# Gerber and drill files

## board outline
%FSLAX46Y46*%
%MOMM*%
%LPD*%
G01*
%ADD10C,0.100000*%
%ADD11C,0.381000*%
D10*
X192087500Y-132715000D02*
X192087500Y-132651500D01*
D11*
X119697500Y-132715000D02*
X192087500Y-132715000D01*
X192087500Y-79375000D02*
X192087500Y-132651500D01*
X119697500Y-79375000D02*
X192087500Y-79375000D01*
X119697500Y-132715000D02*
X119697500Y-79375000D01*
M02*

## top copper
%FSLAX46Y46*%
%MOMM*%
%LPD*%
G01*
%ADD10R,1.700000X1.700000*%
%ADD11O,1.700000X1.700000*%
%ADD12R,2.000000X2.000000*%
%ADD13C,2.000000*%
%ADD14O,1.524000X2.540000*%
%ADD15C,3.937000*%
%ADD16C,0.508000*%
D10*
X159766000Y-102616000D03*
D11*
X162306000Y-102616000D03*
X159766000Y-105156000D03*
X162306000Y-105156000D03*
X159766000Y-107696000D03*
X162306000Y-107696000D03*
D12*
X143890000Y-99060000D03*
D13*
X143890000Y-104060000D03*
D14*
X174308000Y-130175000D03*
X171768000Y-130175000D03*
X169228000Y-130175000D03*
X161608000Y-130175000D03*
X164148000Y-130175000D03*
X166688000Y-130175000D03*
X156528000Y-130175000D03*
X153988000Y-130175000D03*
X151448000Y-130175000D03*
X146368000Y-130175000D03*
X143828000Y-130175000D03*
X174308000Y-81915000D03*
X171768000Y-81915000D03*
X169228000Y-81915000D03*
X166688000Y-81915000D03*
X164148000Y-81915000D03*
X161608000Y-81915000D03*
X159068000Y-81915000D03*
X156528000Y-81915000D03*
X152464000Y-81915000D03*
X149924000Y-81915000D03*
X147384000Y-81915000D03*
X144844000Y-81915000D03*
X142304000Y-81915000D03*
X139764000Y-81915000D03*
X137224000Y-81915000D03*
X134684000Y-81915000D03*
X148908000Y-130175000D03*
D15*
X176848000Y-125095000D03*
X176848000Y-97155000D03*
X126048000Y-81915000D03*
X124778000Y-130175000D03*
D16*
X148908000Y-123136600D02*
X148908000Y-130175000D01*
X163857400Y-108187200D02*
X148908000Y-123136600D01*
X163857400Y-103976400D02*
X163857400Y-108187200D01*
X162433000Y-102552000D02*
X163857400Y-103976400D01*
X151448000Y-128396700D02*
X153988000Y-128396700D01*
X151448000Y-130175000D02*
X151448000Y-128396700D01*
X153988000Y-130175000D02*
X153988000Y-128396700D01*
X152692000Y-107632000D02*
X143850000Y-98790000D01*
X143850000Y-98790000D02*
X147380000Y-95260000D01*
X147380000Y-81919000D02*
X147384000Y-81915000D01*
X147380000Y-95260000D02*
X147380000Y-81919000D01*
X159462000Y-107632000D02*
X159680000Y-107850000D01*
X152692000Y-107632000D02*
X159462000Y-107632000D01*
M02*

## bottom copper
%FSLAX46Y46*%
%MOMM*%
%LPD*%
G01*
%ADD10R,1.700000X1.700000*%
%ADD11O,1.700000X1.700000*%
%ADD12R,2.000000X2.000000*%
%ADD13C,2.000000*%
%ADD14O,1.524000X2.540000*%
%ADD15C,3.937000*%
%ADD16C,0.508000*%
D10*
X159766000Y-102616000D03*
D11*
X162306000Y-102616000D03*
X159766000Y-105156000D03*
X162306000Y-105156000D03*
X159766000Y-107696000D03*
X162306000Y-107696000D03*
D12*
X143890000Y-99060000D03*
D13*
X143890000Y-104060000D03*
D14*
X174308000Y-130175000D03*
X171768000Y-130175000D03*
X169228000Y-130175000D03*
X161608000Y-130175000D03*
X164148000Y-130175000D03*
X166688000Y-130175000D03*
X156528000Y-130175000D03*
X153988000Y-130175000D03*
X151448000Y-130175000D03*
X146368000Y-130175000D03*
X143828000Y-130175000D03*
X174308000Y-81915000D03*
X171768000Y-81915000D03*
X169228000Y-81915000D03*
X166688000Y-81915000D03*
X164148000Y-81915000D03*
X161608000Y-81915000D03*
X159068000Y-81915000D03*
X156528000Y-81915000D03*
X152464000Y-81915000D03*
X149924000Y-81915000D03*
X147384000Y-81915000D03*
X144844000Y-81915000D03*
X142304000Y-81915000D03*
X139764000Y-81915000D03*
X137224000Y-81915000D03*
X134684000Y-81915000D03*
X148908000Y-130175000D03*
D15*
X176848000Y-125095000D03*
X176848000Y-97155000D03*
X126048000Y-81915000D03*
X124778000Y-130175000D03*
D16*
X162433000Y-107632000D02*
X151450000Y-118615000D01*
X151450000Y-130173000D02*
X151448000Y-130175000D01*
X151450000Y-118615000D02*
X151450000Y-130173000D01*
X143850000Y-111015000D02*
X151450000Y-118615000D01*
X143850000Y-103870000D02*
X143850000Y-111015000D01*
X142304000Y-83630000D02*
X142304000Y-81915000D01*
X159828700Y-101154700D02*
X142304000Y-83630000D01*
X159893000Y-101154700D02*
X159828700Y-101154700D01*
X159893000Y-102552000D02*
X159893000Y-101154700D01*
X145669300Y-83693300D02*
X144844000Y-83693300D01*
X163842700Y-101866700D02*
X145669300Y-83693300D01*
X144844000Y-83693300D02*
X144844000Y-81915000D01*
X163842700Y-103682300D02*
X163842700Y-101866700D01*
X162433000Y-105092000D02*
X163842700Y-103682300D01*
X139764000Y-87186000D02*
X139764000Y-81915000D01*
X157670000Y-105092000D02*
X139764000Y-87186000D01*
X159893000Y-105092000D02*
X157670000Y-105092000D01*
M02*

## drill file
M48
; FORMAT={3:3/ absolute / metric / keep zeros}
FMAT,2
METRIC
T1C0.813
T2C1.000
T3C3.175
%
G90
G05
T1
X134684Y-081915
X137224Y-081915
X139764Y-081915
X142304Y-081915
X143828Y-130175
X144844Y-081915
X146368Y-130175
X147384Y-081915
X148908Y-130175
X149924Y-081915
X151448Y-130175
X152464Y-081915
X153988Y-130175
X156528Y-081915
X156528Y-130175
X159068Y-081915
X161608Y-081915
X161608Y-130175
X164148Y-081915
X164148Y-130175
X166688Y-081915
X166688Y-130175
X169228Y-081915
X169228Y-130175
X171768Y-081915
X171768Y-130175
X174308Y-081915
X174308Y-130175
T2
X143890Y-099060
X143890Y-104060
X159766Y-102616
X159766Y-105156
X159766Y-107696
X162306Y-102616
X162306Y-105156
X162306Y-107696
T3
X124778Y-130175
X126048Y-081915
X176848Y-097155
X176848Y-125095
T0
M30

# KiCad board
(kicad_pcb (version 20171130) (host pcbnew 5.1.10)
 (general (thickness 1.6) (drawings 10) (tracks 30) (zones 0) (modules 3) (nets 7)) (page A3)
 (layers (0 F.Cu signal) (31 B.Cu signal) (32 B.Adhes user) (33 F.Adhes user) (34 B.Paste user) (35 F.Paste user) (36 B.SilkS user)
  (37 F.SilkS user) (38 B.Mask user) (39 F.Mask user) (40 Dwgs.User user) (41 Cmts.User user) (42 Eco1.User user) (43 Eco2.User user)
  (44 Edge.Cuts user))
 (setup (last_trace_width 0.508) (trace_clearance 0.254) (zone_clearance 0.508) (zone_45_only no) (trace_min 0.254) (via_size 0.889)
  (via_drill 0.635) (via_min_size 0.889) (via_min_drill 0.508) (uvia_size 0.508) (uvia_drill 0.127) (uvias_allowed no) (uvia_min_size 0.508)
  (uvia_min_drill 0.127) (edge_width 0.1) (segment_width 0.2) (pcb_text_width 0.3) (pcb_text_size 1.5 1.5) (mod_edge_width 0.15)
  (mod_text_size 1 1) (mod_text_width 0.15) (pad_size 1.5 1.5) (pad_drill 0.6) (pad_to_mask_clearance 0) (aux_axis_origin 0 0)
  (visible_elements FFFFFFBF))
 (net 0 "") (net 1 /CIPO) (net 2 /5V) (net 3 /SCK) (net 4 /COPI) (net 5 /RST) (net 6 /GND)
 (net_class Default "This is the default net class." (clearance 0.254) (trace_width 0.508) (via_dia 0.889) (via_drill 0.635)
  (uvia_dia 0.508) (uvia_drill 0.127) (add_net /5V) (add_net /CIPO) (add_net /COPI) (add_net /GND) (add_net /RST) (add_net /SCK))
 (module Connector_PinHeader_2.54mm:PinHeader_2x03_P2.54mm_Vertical (layer F.Cu) (at 159.766 102.616)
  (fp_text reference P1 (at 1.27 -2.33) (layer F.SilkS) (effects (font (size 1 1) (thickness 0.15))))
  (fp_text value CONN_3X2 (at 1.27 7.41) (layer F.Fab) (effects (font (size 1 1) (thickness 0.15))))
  (pad 1 thru_hole rect (at 0 0) (size 1.7 1.7) (drill 1) (layers *.Cu *.Mask) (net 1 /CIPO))
  (pad 2 thru_hole oval (at 2.54 0) (size 1.7 1.7) (drill 1) (layers *.Cu *.Mask) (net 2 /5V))
  (pad 3 thru_hole oval (at 0 2.54) (size 1.7 1.7) (drill 1) (layers *.Cu *.Mask) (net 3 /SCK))
  (pad 4 thru_hole oval (at 2.54 2.54) (size 1.7 1.7) (drill 1) (layers *.Cu *.Mask) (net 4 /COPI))
  (pad 5 thru_hole oval (at 0 5.08) (size 1.7 1.7) (drill 1) (layers *.Cu *.Mask) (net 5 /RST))
  (pad 6 thru_hole oval (at 2.54 5.08) (size 1.7 1.7) (drill 1) (layers *.Cu *.Mask) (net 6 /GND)))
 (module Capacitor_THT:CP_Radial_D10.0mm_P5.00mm (layer F.Cu) (at 143.89 99.06 270)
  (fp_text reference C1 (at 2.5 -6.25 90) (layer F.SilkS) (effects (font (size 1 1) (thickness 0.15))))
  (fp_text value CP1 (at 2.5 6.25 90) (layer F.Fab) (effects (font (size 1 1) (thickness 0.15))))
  (pad 1 thru_hole rect (at 0 0 270) (size 2 2) (drill 1) (layers *.Cu *.Mask) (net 5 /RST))
  (pad 2 thru_hole circle (at 5 0 270) (size 2 2) (drill 1) (layers *.Cu *.Mask) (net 6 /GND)))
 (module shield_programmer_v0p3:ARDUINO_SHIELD (layer F.Cu) (at 119.698 132.715)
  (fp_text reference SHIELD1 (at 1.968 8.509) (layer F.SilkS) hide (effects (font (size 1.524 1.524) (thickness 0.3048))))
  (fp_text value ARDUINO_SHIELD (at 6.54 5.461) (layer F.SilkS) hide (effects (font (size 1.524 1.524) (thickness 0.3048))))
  (pad AD5 thru_hole oval (at 54.61 -2.54 90) (size 2.54 1.524) (drill 0.8128) (layers *.Cu *.Mask F.SilkS))
  (pad AD4 thru_hole oval (at 52.07 -2.54 90) (size 2.54 1.524) (drill 0.8128) (layers *.Cu *.Mask F.SilkS))
  (pad AD3 thru_hole oval (at 49.53 -2.54 90) (size 2.54 1.524) (drill 0.8128) (layers *.Cu *.Mask F.SilkS))
  (pad AD0 thru_hole oval (at 41.91 -2.54 90) (size 2.54 1.524) (drill 0.8128) (layers *.Cu *.Mask F.SilkS))
  (pad AD1 thru_hole oval (at 44.45 -2.54 90) (size 2.54 1.524) (drill 0.8128) (layers *.Cu *.Mask F.SilkS))
  (pad AD2 thru_hole oval (at 46.99 -2.54 90) (size 2.54 1.524) (drill 0.8128) (layers *.Cu *.Mask F.SilkS))
  (pad V_IN thru_hole oval (at 36.83 -2.54 90) (size 2.54 1.524) (drill 0.8128) (layers *.Cu *.Mask F.SilkS))
  (pad GND2 thru_hole oval (at 34.29 -2.54 90) (size 2.54 1.524) (drill 0.8128) (layers *.Cu *.Mask F.SilkS) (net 6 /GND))
  (pad GND1 thru_hole oval (at 31.75 -2.54 90) (size 2.54 1.524) (drill 0.8128) (layers *.Cu *.Mask F.SilkS) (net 6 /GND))
  (pad 3V3 thru_hole oval (at 26.67 -2.54 90) (size 2.54 1.524) (drill 0.8128) (layers *.Cu *.Mask F.SilkS))
  (pad RST thru_hole oval (at 24.13 -2.54 90) (size 2.54 1.524) (drill 0.8128) (layers *.Cu *.Mask F.SilkS))
  (pad 0 thru_hole oval (at 54.61 -50.8 90) (size 2.54 1.524) (drill 0.8128) (layers *.Cu *.Mask F.SilkS))
  (pad 1 thru_hole oval (at 52.07 -50.8 90) (size 2.54 1.524) (drill 0.8128) (layers *.Cu *.Mask F.SilkS))
  (pad 2 thru_hole oval (at 49.53 -50.8 90) (size 2.54 1.524) (drill 0.8128) (layers *.Cu *.Mask F.SilkS))
  (pad 3 thru_hole oval (at 46.99 -50.8 90) (size 2.54 1.524) (drill 0.8128) (layers *.Cu *.Mask F.SilkS))
  (pad 4 thru_hole oval (at 44.45 -50.8 90) (size 2.54 1.524) (drill 0.8128) (layers *.Cu *.Mask F.SilkS))
  (pad 5 thru_hole oval (at 41.91 -50.8 90) (size 2.54 1.524) (drill 0.8128) (layers *.Cu *.Mask F.SilkS))
  (pad 6 thru_hole oval (at 39.37 -50.8 90) (size 2.54 1.524) (drill 0.8128) (layers *.Cu *.Mask F.SilkS))
  (pad 7 thru_hole oval (at 36.83 -50.8 90) (size 2.54 1.524) (drill 0.8128) (layers *.Cu *.Mask F.SilkS))
  (pad 8 thru_hole oval (at 32.766 -50.8 90) (size 2.54 1.524) (drill 0.8128) (layers *.Cu *.Mask F.SilkS))
  (pad 9 thru_hole oval (at 30.226 -50.8 90) (size 2.54 1.524) (drill 0.8128) (layers *.Cu *.Mask F.SilkS))
  (pad 10 thru_hole oval (at 27.686 -50.8 90) (size 2.54 1.524) (drill 0.8128) (layers *.Cu *.Mask F.SilkS) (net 5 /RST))
  (pad 11 thru_hole oval (at 25.146 -50.8 90) (size 2.54 1.524) (drill 0.8128) (layers *.Cu *.Mask F.SilkS) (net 4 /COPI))
  (pad 12 thru_hole oval (at 22.606 -50.8 90) (size 2.54 1.524) (drill 0.8128) (layers *.Cu *.Mask F.SilkS) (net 1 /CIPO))
  (pad 13 thru_hole oval (at 20.066 -50.8 90) (size 2.54 1.524) (drill 0.8128) (layers *.Cu *.Mask F.SilkS) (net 3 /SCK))
  (pad GND3 thru_hole oval (at 17.526 -50.8 90) (size 2.54 1.524) (drill 0.8128) (layers *.Cu *.Mask F.SilkS))
  (pad AREF thru_hole oval (at 14.986 -50.8 90) (size 2.54 1.524) (drill 0.8128) (layers *.Cu *.Mask F.SilkS))
  (pad 5V thru_hole oval (at 29.21 -2.54 90) (size 2.54 1.524) (drill 0.8128) (layers *.Cu *.Mask F.SilkS) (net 2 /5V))
  (pad "" thru_hole circle (at 57.15 -7.62 90) (size 3.937 3.937) (drill 3.175) (layers *.Cu *.Mask F.SilkS))
  (pad "" thru_hole circle (at 57.15 -35.56 90) (size 3.937 3.937) (drill 3.175) (layers *.Cu *.Mask F.SilkS))
  (pad "" thru_hole circle (at 6.35 -50.8 90) (size 3.937 3.937) (drill 3.175) (layers *.Cu *.Mask F.SilkS))
  (pad "" thru_hole circle (at 5.08 -2.54 90) (size 3.937 3.937) (drill 3.175) (layers *.Cu *.Mask F.SilkS)))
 (gr_line (start 192.0875 132.715) (end 192.0875 132.6515) (angle 90) (layer Edge.Cuts) (width 0.1))
 (gr_line (start 119.6975 132.715) (end 192.0875 132.715) (angle 90) (layer Edge.Cuts) (width 0.381))
 (gr_line (start 192.0875 79.375) (end 192.0875 132.6515) (angle 90) (layer Edge.Cuts) (width 0.381))
 (gr_line (start 119.6975 79.375) (end 192.0875 79.375) (angle 90) (layer Edge.Cuts) (width 0.381))
 (gr_line (start 119.6975 132.715) (end 119.6975 79.375) (angle 90) (layer Edge.Cuts) (width 0.381))
 (segment (start 148.908 123.1366) (end 148.908 130.175) (width 0.508) (layer F.Cu) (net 2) (status 20))
 (segment (start 163.8574 108.1872) (end 148.908 123.1366) (width 0.508) (layer F.Cu) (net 2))
 (segment (start 163.8574 103.9764) (end 163.8574 108.1872) (width 0.508) (layer F.Cu) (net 2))
 (segment (start 162.433 102.552) (end 163.8574 103.9764) (width 0.508) (layer F.Cu) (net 2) (status 10))
 (segment (start 151.448 128.3967) (end 153.988 128.3967) (width 0.508) (layer F.Cu) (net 6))
 (segment (start 151.448 130.175) (end 151.448 128.3967) (width 0.508) (layer F.Cu) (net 6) (status 10))
 (segment (start 153.988 130.175) (end 153.988 128.3967) (width 0.508) (layer F.Cu) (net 6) (status 10))
 (segment (start 162.433 107.632) (end 151.45 118.615) (width 0.508) (layer B.Cu) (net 6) (status 10))
 (segment (start 151.45 130.173) (end 151.448 130.175) (width 0.508) (layer B.Cu) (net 6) (status 30))
 (segment (start 151.45 118.615) (end 151.45 130.173) (width 0.508) (layer B.Cu) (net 6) (status 20))
 (segment (start 143.85 111.015) (end 151.45 118.615) (width 0.508) (layer B.Cu) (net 6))
 (segment (start 143.85 103.87) (end 143.85 111.015) (width 0.508) (layer B.Cu) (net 6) (status 10))
 (segment (start 142.304 83.63) (end 142.304 81.915) (width 0.508) (layer B.Cu) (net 1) (status 20))
 (segment (start 159.8287 101.1547) (end 142.304 83.63) (width 0.508) (layer B.Cu) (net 1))
 (segment (start 159.893 101.1547) (end 159.8287 101.1547) (width 0.508) (layer B.Cu) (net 1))
 (segment (start 159.893 102.552) (end 159.893 101.1547) (width 0.508) (layer B.Cu) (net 1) (status 10))
 (segment (start 145.6693 83.6933) (end 144.844 83.6933) (width 0.508) (layer B.Cu) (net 4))
 (segment (start 163.8427 101.8667) (end 145.6693 83.6933) (width 0.508) (layer B.Cu) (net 4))
 (segment (start 144.844 83.6933) (end 144.844 81.915) (width 0.508) (layer B.Cu) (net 4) (status 20))
 (segment (start 163.8427 103.6823) (end 163.8427 101.8667) (width 0.508) (layer B.Cu) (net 4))
 (segment (start 162.433 105.092) (end 163.8427 103.6823) (width 0.508) (layer B.Cu) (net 4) (status 10))
 (segment (start 152.692 107.632) (end 143.85 98.79) (width 0.508) (layer F.Cu) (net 5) (status 20))
 (segment (start 143.85 98.79) (end 147.38 95.26) (width 0.508) (layer F.Cu) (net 5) (status 10))
 (segment (start 147.38 81.919) (end 147.384 81.915) (width 0.508) (layer F.Cu) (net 5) (status 30))
 (segment (start 147.38 95.26) (end 147.38 81.919) (width 0.508) (layer F.Cu) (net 5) (status 20))
 (segment (start 159.462 107.632) (end 159.68 107.85) (width 0.508) (layer F.Cu) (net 5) (status 30))
 (segment (start 152.692 107.632) (end 159.462 107.632) (width 0.508) (layer F.Cu) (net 5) (status 20))
 (segment (start 139.764 87.186) (end 139.764 81.915) (width 0.508) (layer B.Cu) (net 3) (status 20))
 (segment (start 157.67 105.092) (end 139.764 87.186) (width 0.508) (layer B.Cu) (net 3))
 (segment (start 159.893 105.092) (end 157.67 105.092) (width 0.508) (layer B.Cu) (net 3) (status 10)))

